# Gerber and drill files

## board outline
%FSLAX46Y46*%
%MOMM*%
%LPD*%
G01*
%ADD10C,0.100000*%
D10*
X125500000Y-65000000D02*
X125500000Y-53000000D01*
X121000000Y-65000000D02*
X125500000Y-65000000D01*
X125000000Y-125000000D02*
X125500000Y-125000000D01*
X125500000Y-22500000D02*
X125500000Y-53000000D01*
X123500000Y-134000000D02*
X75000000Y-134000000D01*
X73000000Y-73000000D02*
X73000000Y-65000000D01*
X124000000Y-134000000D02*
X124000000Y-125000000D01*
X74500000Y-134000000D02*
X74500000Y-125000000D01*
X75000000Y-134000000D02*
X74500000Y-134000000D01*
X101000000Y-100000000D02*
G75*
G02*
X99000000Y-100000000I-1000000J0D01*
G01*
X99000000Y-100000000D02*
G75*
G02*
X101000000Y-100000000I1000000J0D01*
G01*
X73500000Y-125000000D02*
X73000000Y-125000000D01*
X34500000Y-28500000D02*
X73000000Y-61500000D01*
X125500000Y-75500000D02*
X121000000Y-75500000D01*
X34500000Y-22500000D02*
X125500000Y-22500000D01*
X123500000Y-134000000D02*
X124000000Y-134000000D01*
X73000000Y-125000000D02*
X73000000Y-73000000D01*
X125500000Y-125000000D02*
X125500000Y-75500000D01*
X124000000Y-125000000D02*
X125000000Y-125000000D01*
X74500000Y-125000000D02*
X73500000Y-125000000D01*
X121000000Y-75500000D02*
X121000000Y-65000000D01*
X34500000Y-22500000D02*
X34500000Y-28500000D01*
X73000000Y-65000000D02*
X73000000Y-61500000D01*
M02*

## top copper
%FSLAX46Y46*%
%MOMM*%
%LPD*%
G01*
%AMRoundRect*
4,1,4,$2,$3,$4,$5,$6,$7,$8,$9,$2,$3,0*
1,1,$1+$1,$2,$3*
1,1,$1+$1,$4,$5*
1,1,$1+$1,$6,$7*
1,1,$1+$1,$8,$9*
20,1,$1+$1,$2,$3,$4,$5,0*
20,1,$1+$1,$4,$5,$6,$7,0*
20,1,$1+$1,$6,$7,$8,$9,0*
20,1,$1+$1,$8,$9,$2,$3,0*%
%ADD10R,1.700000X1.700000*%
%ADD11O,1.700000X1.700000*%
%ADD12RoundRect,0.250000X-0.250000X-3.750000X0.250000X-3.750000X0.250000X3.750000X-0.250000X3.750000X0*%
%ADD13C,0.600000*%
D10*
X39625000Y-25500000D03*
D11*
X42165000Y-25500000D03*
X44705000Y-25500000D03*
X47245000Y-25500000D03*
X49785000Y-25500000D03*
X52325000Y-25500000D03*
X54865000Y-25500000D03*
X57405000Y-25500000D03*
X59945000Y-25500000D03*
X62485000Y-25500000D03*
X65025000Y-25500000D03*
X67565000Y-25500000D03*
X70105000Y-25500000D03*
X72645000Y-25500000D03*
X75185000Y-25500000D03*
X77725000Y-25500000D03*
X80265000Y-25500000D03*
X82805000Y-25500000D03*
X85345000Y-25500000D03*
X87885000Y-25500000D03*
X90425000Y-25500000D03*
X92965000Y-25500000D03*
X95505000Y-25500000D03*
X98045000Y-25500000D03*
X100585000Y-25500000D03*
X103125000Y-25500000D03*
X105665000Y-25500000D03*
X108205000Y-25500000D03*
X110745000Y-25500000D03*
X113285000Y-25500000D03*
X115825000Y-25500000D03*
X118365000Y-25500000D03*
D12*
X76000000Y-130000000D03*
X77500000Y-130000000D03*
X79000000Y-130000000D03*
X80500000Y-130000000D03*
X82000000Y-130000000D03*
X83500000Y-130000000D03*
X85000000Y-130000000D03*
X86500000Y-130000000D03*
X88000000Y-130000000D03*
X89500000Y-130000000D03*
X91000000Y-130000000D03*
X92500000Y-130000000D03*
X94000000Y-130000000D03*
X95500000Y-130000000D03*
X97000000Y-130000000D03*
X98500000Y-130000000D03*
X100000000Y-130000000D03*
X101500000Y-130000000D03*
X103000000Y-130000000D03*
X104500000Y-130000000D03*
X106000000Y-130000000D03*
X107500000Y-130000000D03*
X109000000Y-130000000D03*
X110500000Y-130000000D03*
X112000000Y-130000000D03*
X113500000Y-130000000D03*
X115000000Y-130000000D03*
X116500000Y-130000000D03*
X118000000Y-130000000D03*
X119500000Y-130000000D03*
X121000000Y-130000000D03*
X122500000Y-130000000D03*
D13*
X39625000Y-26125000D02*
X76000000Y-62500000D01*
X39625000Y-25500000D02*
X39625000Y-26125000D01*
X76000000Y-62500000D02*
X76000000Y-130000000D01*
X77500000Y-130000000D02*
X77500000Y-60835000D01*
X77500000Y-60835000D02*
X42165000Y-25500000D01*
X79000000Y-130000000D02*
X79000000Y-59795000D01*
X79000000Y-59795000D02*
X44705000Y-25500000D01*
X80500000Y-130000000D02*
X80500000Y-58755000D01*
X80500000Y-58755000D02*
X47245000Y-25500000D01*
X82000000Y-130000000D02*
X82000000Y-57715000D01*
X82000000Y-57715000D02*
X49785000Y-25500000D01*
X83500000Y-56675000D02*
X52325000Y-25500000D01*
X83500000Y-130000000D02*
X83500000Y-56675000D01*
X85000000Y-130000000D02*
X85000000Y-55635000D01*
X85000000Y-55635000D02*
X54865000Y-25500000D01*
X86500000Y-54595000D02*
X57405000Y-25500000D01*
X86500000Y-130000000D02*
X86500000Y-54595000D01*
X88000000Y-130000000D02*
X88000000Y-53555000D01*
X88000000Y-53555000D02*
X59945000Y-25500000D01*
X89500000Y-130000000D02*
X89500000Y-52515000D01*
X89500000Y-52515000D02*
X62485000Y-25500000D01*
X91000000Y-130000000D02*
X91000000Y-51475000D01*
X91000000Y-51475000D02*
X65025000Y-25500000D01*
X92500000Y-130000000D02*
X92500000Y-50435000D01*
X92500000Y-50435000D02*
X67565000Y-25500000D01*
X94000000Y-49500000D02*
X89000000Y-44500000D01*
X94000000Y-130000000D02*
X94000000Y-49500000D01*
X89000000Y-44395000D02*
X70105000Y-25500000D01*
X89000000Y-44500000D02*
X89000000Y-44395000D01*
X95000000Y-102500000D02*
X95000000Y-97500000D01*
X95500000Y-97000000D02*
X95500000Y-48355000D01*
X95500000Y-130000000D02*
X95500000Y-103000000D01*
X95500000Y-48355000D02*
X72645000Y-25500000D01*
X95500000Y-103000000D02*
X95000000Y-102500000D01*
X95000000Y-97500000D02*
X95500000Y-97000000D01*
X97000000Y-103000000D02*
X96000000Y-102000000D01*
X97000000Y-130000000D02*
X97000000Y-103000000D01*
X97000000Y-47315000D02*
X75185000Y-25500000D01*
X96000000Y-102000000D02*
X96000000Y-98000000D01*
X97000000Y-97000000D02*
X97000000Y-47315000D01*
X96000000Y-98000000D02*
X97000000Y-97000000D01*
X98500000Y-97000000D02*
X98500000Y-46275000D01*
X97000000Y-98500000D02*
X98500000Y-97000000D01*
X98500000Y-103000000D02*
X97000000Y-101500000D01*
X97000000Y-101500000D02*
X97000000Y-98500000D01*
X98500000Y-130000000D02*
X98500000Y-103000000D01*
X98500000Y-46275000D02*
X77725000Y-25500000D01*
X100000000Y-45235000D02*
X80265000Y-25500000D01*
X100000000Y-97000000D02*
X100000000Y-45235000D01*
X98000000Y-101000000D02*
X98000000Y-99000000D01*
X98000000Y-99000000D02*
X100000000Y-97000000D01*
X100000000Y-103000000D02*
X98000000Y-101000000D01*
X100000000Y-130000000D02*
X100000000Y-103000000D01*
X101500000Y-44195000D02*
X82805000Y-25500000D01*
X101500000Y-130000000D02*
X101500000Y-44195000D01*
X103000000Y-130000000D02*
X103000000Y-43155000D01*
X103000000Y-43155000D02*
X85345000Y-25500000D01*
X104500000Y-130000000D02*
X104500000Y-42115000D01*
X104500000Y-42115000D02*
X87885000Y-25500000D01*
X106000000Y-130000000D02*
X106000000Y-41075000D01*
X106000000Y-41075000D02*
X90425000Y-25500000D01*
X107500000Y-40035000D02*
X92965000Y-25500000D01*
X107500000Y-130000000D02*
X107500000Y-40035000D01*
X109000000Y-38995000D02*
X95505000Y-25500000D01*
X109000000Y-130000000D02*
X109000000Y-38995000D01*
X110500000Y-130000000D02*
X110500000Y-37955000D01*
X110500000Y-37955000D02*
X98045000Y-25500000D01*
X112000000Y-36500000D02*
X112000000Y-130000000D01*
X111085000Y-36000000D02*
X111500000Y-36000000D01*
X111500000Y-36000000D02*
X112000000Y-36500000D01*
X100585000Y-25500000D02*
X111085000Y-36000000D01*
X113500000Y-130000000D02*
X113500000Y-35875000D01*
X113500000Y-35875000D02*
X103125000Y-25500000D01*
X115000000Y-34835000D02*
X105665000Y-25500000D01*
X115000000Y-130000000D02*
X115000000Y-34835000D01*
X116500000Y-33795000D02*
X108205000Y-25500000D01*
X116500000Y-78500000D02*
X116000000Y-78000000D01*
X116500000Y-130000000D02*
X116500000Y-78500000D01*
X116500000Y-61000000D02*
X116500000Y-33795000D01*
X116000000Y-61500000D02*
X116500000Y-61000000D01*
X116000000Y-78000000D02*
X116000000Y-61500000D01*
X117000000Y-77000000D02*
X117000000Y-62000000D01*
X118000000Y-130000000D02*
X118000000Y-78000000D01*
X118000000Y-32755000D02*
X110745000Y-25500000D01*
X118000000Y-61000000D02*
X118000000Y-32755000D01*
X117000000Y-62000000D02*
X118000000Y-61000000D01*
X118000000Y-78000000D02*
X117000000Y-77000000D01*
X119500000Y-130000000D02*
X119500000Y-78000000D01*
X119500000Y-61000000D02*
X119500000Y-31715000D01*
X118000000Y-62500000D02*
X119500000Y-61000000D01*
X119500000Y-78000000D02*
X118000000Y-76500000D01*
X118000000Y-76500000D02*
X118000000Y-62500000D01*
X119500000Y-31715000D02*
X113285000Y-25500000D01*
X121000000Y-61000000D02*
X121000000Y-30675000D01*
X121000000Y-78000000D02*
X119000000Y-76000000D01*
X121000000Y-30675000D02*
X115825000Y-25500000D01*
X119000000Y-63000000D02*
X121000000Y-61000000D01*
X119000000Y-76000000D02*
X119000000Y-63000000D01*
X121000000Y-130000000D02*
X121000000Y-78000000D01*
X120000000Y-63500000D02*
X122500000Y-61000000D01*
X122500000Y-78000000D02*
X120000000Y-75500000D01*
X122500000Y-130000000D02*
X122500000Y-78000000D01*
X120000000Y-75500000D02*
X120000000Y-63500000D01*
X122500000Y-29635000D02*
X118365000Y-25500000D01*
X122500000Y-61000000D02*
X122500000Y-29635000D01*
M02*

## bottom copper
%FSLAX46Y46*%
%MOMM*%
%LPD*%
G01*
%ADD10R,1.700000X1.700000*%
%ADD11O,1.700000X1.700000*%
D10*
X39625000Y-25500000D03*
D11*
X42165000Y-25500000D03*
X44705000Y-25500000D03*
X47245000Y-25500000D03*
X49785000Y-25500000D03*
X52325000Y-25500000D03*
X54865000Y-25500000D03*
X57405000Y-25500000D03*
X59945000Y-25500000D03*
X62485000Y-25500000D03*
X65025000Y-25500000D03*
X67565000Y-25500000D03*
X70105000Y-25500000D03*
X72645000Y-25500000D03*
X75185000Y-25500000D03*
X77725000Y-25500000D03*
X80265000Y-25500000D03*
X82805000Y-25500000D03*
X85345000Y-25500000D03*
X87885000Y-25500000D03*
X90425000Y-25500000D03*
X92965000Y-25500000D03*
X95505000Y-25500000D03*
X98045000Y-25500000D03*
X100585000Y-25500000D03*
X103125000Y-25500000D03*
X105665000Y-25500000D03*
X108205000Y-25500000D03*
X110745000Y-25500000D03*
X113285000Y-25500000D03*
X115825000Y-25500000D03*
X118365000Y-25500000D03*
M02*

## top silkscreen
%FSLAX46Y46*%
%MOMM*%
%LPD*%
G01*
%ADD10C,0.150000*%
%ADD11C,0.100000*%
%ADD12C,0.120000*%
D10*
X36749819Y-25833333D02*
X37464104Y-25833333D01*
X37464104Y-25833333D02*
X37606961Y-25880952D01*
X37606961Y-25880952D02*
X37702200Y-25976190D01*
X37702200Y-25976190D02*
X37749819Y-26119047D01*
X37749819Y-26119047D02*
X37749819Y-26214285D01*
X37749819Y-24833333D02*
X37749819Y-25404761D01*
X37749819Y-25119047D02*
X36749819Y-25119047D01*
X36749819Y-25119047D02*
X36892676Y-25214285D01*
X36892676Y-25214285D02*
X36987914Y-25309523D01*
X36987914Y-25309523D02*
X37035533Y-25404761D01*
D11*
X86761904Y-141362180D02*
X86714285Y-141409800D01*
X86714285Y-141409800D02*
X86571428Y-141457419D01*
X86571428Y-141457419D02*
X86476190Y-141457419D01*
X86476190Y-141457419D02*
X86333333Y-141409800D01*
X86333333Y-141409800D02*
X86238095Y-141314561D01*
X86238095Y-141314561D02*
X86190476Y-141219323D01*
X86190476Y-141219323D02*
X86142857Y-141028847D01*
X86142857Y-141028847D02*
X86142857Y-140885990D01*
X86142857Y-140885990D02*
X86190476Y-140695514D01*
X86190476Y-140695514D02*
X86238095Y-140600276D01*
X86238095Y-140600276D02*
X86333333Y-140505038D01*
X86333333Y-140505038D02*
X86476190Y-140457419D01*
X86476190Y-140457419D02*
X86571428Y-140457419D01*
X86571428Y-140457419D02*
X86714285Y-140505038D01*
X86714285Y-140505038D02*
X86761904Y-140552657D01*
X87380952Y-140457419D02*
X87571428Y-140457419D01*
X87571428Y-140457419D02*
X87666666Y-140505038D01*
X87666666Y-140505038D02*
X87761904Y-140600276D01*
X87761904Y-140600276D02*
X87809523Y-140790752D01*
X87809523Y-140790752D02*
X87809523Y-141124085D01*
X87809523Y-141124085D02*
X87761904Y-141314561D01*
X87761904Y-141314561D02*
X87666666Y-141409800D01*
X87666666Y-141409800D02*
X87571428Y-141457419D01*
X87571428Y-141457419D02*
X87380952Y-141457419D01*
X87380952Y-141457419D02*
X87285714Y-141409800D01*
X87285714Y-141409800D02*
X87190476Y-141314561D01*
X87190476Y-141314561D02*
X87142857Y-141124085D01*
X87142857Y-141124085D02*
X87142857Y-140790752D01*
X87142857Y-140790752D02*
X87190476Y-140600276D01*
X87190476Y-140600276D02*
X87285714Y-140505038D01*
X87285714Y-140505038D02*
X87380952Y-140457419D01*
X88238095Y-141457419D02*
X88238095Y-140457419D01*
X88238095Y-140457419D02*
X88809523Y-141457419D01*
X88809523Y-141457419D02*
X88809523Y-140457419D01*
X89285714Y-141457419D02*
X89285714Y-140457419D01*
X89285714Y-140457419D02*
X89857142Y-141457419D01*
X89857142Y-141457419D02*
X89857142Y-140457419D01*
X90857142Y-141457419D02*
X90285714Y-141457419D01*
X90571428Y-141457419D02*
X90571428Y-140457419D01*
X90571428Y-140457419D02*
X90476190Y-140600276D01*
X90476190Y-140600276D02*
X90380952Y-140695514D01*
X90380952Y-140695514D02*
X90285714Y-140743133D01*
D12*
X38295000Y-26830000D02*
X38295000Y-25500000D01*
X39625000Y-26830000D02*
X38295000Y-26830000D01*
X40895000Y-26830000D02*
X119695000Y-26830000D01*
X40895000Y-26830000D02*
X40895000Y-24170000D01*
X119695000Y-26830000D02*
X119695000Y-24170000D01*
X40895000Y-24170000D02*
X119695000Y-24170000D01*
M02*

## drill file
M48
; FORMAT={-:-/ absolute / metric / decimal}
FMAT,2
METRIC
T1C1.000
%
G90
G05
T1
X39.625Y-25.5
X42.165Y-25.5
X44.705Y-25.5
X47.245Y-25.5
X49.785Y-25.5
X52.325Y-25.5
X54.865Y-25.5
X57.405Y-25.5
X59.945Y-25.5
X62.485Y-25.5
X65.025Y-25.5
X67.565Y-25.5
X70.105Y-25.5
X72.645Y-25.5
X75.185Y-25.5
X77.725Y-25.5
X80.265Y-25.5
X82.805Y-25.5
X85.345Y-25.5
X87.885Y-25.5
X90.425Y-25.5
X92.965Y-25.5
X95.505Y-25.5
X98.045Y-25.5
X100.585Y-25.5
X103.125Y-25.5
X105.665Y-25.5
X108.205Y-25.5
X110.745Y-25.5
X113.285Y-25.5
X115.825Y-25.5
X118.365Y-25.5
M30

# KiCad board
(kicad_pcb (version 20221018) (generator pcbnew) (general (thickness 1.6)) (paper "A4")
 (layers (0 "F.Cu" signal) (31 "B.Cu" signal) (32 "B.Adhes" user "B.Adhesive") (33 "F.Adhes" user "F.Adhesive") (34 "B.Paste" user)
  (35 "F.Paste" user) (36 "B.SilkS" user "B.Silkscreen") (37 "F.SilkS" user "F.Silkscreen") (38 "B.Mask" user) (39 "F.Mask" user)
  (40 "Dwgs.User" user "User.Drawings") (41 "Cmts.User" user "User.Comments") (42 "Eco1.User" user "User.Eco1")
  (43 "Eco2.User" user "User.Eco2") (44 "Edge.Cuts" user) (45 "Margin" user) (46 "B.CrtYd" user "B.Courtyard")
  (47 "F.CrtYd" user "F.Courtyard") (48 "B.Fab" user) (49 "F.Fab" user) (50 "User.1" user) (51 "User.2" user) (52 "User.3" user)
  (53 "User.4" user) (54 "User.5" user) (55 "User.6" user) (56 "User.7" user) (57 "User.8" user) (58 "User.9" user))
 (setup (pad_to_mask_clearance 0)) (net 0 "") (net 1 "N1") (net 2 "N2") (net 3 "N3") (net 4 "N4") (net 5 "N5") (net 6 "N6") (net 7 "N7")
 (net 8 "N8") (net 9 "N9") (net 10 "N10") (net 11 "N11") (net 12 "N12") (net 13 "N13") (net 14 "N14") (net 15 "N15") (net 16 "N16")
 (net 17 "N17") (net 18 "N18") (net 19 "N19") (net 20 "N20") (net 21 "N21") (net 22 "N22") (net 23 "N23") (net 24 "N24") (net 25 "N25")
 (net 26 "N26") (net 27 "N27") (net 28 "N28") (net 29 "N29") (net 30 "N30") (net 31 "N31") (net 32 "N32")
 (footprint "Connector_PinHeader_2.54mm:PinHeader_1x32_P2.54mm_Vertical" (layer "F.Cu") (at 39.625 25.5 90)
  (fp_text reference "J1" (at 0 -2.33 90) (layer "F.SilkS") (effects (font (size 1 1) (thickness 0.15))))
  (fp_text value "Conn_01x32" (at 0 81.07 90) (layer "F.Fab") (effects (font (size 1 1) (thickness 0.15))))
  (fp_line (start -1.33 -1.33) (end 0 -1.33) (stroke (width 0.12) (type solid)) (layer "F.SilkS"))
  (fp_line (start -1.33 0) (end -1.33 -1.33) (stroke (width 0.12) (type solid)) (layer "F.SilkS"))
  (fp_line (start -1.33 1.27) (end -1.33 80.07) (stroke (width 0.12) (type solid)) (layer "F.SilkS"))
  (fp_line (start -1.33 1.27) (end 1.33 1.27) (stroke (width 0.12) (type solid)) (layer "F.SilkS"))
  (fp_line (start -1.33 80.07) (end 1.33 80.07) (stroke (width 0.12) (type solid)) (layer "F.SilkS"))
  (fp_line (start 1.33 1.27) (end 1.33 80.07) (stroke (width 0.12) (type solid)) (layer "F.SilkS"))
  (pad "1" thru_hole rect (at 0 0 90) (size 1.7 1.7) (drill 1) (layers "*.Cu" "*.Mask") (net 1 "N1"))
  (pad "2" thru_hole oval (at 0 2.54 90) (size 1.7 1.7) (drill 1) (layers "*.Cu" "*.Mask") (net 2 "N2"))
  (pad "3" thru_hole oval (at 0 5.08 90) (size 1.7 1.7) (drill 1) (layers "*.Cu" "*.Mask") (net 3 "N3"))
  (pad "4" thru_hole oval (at 0 7.62 90) (size 1.7 1.7) (drill 1) (layers "*.Cu" "*.Mask") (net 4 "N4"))
  (pad "5" thru_hole oval (at 0 10.16 90) (size 1.7 1.7) (drill 1) (layers "*.Cu" "*.Mask") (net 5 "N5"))
  (pad "6" thru_hole oval (at 0 12.7 90) (size 1.7 1.7) (drill 1) (layers "*.Cu" "*.Mask") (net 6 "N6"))
  (pad "7" thru_hole oval (at 0 15.24 90) (size 1.7 1.7) (drill 1) (layers "*.Cu" "*.Mask") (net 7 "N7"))
  (pad "8" thru_hole oval (at 0 17.78 90) (size 1.7 1.7) (drill 1) (layers "*.Cu" "*.Mask") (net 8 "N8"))
  (pad "9" thru_hole oval (at 0 20.32 90) (size 1.7 1.7) (drill 1) (layers "*.Cu" "*.Mask") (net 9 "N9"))
  (pad "10" thru_hole oval (at 0 22.86 90) (size 1.7 1.7) (drill 1) (layers "*.Cu" "*.Mask") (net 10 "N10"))
  (pad "11" thru_hole oval (at 0 25.4 90) (size 1.7 1.7) (drill 1) (layers "*.Cu" "*.Mask") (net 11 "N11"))
  (pad "12" thru_hole oval (at 0 27.94 90) (size 1.7 1.7) (drill 1) (layers "*.Cu" "*.Mask") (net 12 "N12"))
  (pad "13" thru_hole oval (at 0 30.48 90) (size 1.7 1.7) (drill 1) (layers "*.Cu" "*.Mask") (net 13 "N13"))
  (pad "14" thru_hole oval (at 0 33.02 90) (size 1.7 1.7) (drill 1) (layers "*.Cu" "*.Mask") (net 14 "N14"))
  (pad "15" thru_hole oval (at 0 35.56 90) (size 1.7 1.7) (drill 1) (layers "*.Cu" "*.Mask") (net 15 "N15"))
  (pad "16" thru_hole oval (at 0 38.1 90) (size 1.7 1.7) (drill 1) (layers "*.Cu" "*.Mask") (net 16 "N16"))
  (pad "17" thru_hole oval (at 0 40.64 90) (size 1.7 1.7) (drill 1) (layers "*.Cu" "*.Mask") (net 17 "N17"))
  (pad "18" thru_hole oval (at 0 43.18 90) (size 1.7 1.7) (drill 1) (layers "*.Cu" "*.Mask") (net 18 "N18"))
  (pad "19" thru_hole oval (at 0 45.72 90) (size 1.7 1.7) (drill 1) (layers "*.Cu" "*.Mask") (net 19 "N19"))
  (pad "20" thru_hole oval (at 0 48.26 90) (size 1.7 1.7) (drill 1) (layers "*.Cu" "*.Mask") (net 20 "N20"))
  (pad "21" thru_hole oval (at 0 50.8 90) (size 1.7 1.7) (drill 1) (layers "*.Cu" "*.Mask") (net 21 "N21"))
  (pad "22" thru_hole oval (at 0 53.34 90) (size 1.7 1.7) (drill 1) (layers "*.Cu" "*.Mask") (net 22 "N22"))
  (pad "23" thru_hole oval (at 0 55.88 90) (size 1.7 1.7) (drill 1) (layers "*.Cu" "*.Mask") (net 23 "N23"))
  (pad "24" thru_hole oval (at 0 58.42 90) (size 1.7 1.7) (drill 1) (layers "*.Cu" "*.Mask") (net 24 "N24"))
  (pad "25" thru_hole oval (at 0 60.96 90) (size 1.7 1.7) (drill 1) (layers "*.Cu" "*.Mask") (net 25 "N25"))
  (pad "26" thru_hole oval (at 0 63.5 90) (size 1.7 1.7) (drill 1) (layers "*.Cu" "*.Mask") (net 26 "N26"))
  (pad "27" thru_hole oval (at 0 66.04 90) (size 1.7 1.7) (drill 1) (layers "*.Cu" "*.Mask") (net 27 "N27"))
  (pad "28" thru_hole oval (at 0 68.58 90) (size 1.7 1.7) (drill 1) (layers "*.Cu" "*.Mask") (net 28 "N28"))
  (pad "29" thru_hole oval (at 0 71.12 90) (size 1.7 1.7) (drill 1) (layers "*.Cu" "*.Mask") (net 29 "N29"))
  (pad "30" thru_hole oval (at 0 73.66 90) (size 1.7 1.7) (drill 1) (layers "*.Cu" "*.Mask") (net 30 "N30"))
  (pad "31" thru_hole oval (at 0 76.2 90) (size 1.7 1.7) (drill 1) (layers "*.Cu" "*.Mask") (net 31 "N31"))
  (pad "32" thru_hole oval (at 0 78.74 90) (size 1.7 1.7) (drill 1) (layers "*.Cu" "*.Mask") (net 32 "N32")))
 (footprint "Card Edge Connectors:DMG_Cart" (layer "F.Cu") (at 75 134)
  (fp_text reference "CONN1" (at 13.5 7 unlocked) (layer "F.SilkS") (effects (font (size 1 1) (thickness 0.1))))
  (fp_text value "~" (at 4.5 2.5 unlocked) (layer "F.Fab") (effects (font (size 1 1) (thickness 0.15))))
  (pad "1" smd roundrect (at 1 -4) (size 1 8) (layers "F.Cu" "F.Paste" "F.Mask") (roundrect_rratio 0.25) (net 1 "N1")
   (thermal_bridge_angle 45))
  (pad "2" smd roundrect (at 2.5 -4) (size 1 8) (layers "F.Cu" "F.Paste" "F.Mask") (roundrect_rratio 0.25) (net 2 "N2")
   (thermal_bridge_angle 45))
  (pad "3" smd roundrect (at 4 -4) (size 1 8) (layers "F.Cu" "F.Paste" "F.Mask") (roundrect_rratio 0.25) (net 3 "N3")
   (thermal_bridge_angle 45))
  (pad "4" smd roundrect (at 5.5 -4) (size 1 8) (layers "F.Cu" "F.Paste" "F.Mask") (roundrect_rratio 0.25) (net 4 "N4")
   (thermal_bridge_angle 45))
  (pad "5" smd roundrect (at 7 -4) (size 1 8) (layers "F.Cu" "F.Paste" "F.Mask") (roundrect_rratio 0.25) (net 5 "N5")
   (thermal_bridge_angle 45))
  (pad "6" smd roundrect (at 8.5 -4) (size 1 8) (layers "F.Cu" "F.Paste" "F.Mask") (roundrect_rratio 0.25) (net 6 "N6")
   (thermal_bridge_angle 45))
  (pad "7" smd roundrect (at 10 -4) (size 1 8) (layers "F.Cu" "F.Paste" "F.Mask") (roundrect_rratio 0.25) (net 7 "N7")
   (thermal_bridge_angle 45))
  (pad "8" smd roundrect (at 11.5 -4) (size 1 8) (layers "F.Cu" "F.Paste" "F.Mask") (roundrect_rratio 0.25) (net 8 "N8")
   (thermal_bridge_angle 45))
  (pad "9" smd roundrect (at 13 -4) (size 1 8) (layers "F.Cu" "F.Paste" "F.Mask") (roundrect_rratio 0.25) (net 9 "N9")
   (thermal_bridge_angle 45))
  (pad "10" smd roundrect (at 14.5 -4) (size 1 8) (layers "F.Cu" "F.Paste" "F.Mask") (roundrect_rratio 0.25) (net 10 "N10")
   (thermal_bridge_angle 45))
  (pad "11" smd roundrect (at 16 -4) (size 1 8) (layers "F.Cu" "F.Paste" "F.Mask") (roundrect_rratio 0.25) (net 11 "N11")
   (thermal_bridge_angle 45))
  (pad "12" smd roundrect (at 17.5 -4) (size 1 8) (layers "F.Cu" "F.Paste" "F.Mask") (roundrect_rratio 0.25) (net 12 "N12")
   (thermal_bridge_angle 45))
  (pad "13" smd roundrect (at 19 -4) (size 1 8) (layers "F.Cu" "F.Paste" "F.Mask") (roundrect_rratio 0.25) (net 13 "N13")
   (thermal_bridge_angle 45))
  (pad "14" smd roundrect (at 20.5 -4) (size 1 8) (layers "F.Cu" "F.Paste" "F.Mask") (roundrect_rratio 0.25) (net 14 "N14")
   (thermal_bridge_angle 45))
  (pad "15" smd roundrect (at 22 -4) (size 1 8) (layers "F.Cu" "F.Paste" "F.Mask") (roundrect_rratio 0.25) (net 15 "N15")
   (thermal_bridge_angle 45))
  (pad "16" smd roundrect (at 23.5 -4) (size 1 8) (layers "F.Cu" "F.Paste" "F.Mask") (roundrect_rratio 0.25) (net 16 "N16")
   (thermal_bridge_angle 45))
  (pad "17" smd roundrect (at 25 -4) (size 1 8) (layers "F.Cu" "F.Paste" "F.Mask") (roundrect_rratio 0.25) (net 17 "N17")
   (thermal_bridge_angle 45))
  (pad "18" smd roundrect (at 26.5 -4) (size 1 8) (layers "F.Cu" "F.Paste" "F.Mask") (roundrect_rratio 0.25) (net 18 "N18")
   (thermal_bridge_angle 45))
  (pad "19" smd roundrect (at 28 -4) (size 1 8) (layers "F.Cu" "F.Paste" "F.Mask") (roundrect_rratio 0.25) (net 19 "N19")
   (thermal_bridge_angle 45))
  (pad "20" smd roundrect (at 29.5 -4) (size 1 8) (layers "F.Cu" "F.Paste" "F.Mask") (roundrect_rratio 0.25) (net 20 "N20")
   (thermal_bridge_angle 45))
  (pad "21" smd roundrect (at 31 -4) (size 1 8) (layers "F.Cu" "F.Paste" "F.Mask") (roundrect_rratio 0.25) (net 21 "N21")
   (thermal_bridge_angle 45))
  (pad "22" smd roundrect (at 32.5 -4) (size 1 8) (layers "F.Cu" "F.Paste" "F.Mask") (roundrect_rratio 0.25) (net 22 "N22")
   (thermal_bridge_angle 45))
  (pad "23" smd roundrect (at 34 -4) (size 1 8) (layers "F.Cu" "F.Paste" "F.Mask") (roundrect_rratio 0.25) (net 23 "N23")
   (thermal_bridge_angle 45))
  (pad "24" smd roundrect (at 35.5 -4) (size 1 8) (layers "F.Cu" "F.Paste" "F.Mask") (roundrect_rratio 0.25) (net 24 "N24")
   (thermal_bridge_angle 45))
  (pad "25" smd roundrect (at 37 -4) (size 1 8) (layers "F.Cu" "F.Paste" "F.Mask") (roundrect_rratio 0.25) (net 25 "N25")
   (thermal_bridge_angle 45))
  (pad "26" smd roundrect (at 38.5 -4) (size 1 8) (layers "F.Cu" "F.Paste" "F.Mask") (roundrect_rratio 0.25) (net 26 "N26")
   (thermal_bridge_angle 45))
  (pad "27" smd roundrect (at 40 -4) (size 1 8) (layers "F.Cu" "F.Paste" "F.Mask") (roundrect_rratio 0.25) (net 27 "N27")
   (thermal_bridge_angle 45))
  (pad "28" smd roundrect (at 41.5 -4) (size 1 8) (layers "F.Cu" "F.Paste" "F.Mask") (roundrect_rratio 0.25) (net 28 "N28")
   (thermal_bridge_angle 45))
  (pad "29" smd roundrect (at 43 -4) (size 1 8) (layers "F.Cu" "F.Paste" "F.Mask") (roundrect_rratio 0.25) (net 29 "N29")
   (thermal_bridge_angle 45))
  (pad "30" smd roundrect (at 44.5 -4) (size 1 8) (layers "F.Cu" "F.Paste" "F.Mask") (roundrect_rratio 0.25) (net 30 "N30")
   (thermal_bridge_angle 45))
  (pad "31" smd roundrect (at 46 -4) (size 1 8) (layers "F.Cu" "F.Paste" "F.Mask") (roundrect_rratio 0.25) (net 31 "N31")
   (thermal_bridge_angle 45))
  (pad "32" smd roundrect (at 47.5 -4) (size 1 8) (layers "F.Cu" "F.Paste" "F.Mask") (roundrect_rratio 0.25) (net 32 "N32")
   (thermal_bridge_angle 45)))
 (gr_line (start 125.5 65) (end 125.5 53) (stroke (width 0.1) (type default)) (layer "Edge.Cuts"))
 (gr_line (start 121 65) (end 125.5 65) (stroke (width 0.1) (type default)) (layer "Edge.Cuts"))
 (gr_line (start 125 125) (end 125.5 125) (stroke (width 0.1) (type default)) (layer "Edge.Cuts"))
 (gr_line (start 125.5 22.5) (end 125.5 53) (stroke (width 0.1) (type default)) (layer "Edge.Cuts"))
 (gr_line (start 123.5 134) (end 75 134) (stroke (width 0.1) (type default)) (layer "Edge.Cuts"))
 (gr_line (start 73 73) (end 73 65) (stroke (width 0.1) (type default)) (layer "Edge.Cuts"))
 (gr_line (start 124 134) (end 124 125) (stroke (width 0.1) (type default)) (layer "Edge.Cuts"))
 (gr_line (start 74.5 134) (end 74.5 125) (stroke (width 0.1) (type default)) (layer "Edge.Cuts"))
 (gr_line (start 75 134) (end 74.5 134) (stroke (width 0.1) (type default)) (layer "Edge.Cuts"))
 (gr_circle (center 100 100) (end 101 100) (stroke (width 0.1) (type default)) (fill none) (layer "Edge.Cuts"))
 (gr_line (start 73.5 125) (end 73 125) (stroke (width 0.1) (type default)) (layer "Edge.Cuts"))
 (gr_line (start 34.5 28.5) (end 73 61.5) (stroke (width 0.1) (type default)) (layer "Edge.Cuts"))
 (gr_line (start 125.5 75.5) (end 121 75.5) (stroke (width 0.1) (type default)) (layer "Edge.Cuts"))
 (gr_line (start 34.5 22.5) (end 125.5 22.5) (stroke (width 0.1) (type default)) (layer "Edge.Cuts"))
 (gr_line (start 123.5 134) (end 124 134) (stroke (width 0.1) (type default)) (layer "Edge.Cuts"))
 (gr_line (start 73 125) (end 73 73) (stroke (width 0.1) (type default)) (layer "Edge.Cuts"))
 (gr_line (start 125.5 125) (end 125.5 75.5) (stroke (width 0.1) (type default)) (layer "Edge.Cuts"))
 (gr_line (start 124 125) (end 125 125) (stroke (width 0.1) (type default)) (layer "Edge.Cuts"))
 (gr_line (start 74.5 125) (end 73.5 125) (stroke (width 0.1) (type default)) (layer "Edge.Cuts"))
 (gr_line (start 121 75.5) (end 121 65) (stroke (width 0.1) (type default)) (layer "Edge.Cuts"))
 (gr_line (start 34.5 22.5) (end 34.5 28.5) (stroke (width 0.1) (type default)) (layer "Edge.Cuts"))
 (gr_line (start 73 65) (end 73 61.5) (stroke (width 0.1) (type default)) (layer "Edge.Cuts"))
 (segment (start 39.625 26.125) (end 76 62.5) (width 0.6) (layer "F.Cu") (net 1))
 (segment (start 39.625 25.5) (end 39.625 26.125) (width 0.6) (layer "F.Cu") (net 1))
 (segment (start 76 62.5) (end 76 130) (width 0.6) (layer "F.Cu") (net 1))
 (segment (start 77.5 130) (end 77.5 60.835) (width 0.6) (layer "F.Cu") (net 2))
 (segment (start 77.5 60.835) (end 42.165 25.5) (width 0.6) (layer "F.Cu") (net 2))
 (segment (start 79 130) (end 79 59.795) (width 0.6) (layer "F.Cu") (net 3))
 (segment (start 79 59.795) (end 44.705 25.5) (width 0.6) (layer "F.Cu") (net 3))
 (segment (start 80.5 130) (end 80.5 58.755) (width 0.6) (layer "F.Cu") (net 4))
 (segment (start 80.5 58.755) (end 47.245 25.5) (width 0.6) (layer "F.Cu") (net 4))
 (segment (start 82 130) (end 82 57.715) (width 0.6) (layer "F.Cu") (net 5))
 (segment (start 82 57.715) (end 49.785 25.5) (width 0.6) (layer "F.Cu") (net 5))
 (segment (start 83.5 56.675) (end 52.325 25.5) (width 0.6) (layer "F.Cu") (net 6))
 (segment (start 83.5 130) (end 83.5 56.675) (width 0.6) (layer "F.Cu") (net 6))
 (segment (start 85 130) (end 85 55.635) (width 0.6) (layer "F.Cu") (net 7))
 (segment (start 85 55.635) (end 54.865 25.5) (width 0.6) (layer "F.Cu") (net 7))
 (segment (start 86.5 54.595) (end 57.405 25.5) (width 0.6) (layer "F.Cu") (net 8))
 (segment (start 86.5 130) (end 86.5 54.595) (width 0.6) (layer "F.Cu") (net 8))
 (segment (start 88 130) (end 88 53.555) (width 0.6) (layer "F.Cu") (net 9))
 (segment (start 88 53.555) (end 59.945 25.5) (width 0.6) (layer "F.Cu") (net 9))
 (segment (start 89.5 130) (end 89.5 52.515) (width 0.6) (layer "F.Cu") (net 10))
 (segment (start 89.5 52.515) (end 62.485 25.5) (width 0.6) (layer "F.Cu") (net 10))
 (segment (start 91 130) (end 91 51.475) (width 0.6) (layer "F.Cu") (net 11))
 (segment (start 91 51.475) (end 65.025 25.5) (width 0.6) (layer "F.Cu") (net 11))
 (segment (start 92.5 130) (end 92.5 50.435) (width 0.6) (layer "F.Cu") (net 12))
 (segment (start 92.5 50.435) (end 67.565 25.5) (width 0.6) (layer "F.Cu") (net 12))
 (segment (start 94 49.5) (end 89 44.5) (width 0.6) (layer "F.Cu") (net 13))
 (segment (start 94 130) (end 94 49.5) (width 0.6) (layer "F.Cu") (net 13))
 (segment (start 89 44.395) (end 70.105 25.5) (width 0.6) (layer "F.Cu") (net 13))
 (segment (start 89 44.5) (end 89 44.395) (width 0.6) (layer "F.Cu") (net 13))
 (segment (start 95 102.5) (end 95 97.5) (width 0.6) (layer "F.Cu") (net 14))
 (segment (start 95.5 97) (end 95.5 48.355) (width 0.6) (layer "F.Cu") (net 14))
 (segment (start 95.5 130) (end 95.5 103) (width 0.6) (layer "F.Cu") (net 14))
 (segment (start 95.5 48.355) (end 72.645 25.5) (width 0.6) (layer "F.Cu") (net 14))
 (segment (start 95.5 103) (end 95 102.5) (width 0.6) (layer "F.Cu") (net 14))
 (segment (start 95 97.5) (end 95.5 97) (width 0.6) (layer "F.Cu") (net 14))
 (segment (start 97 103) (end 96 102) (width 0.6) (layer "F.Cu") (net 15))
 (segment (start 97 130) (end 97 103) (width 0.6) (layer "F.Cu") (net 15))
 (segment (start 97 47.315) (end 75.185 25.5) (width 0.6) (layer "F.Cu") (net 15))
 (segment (start 96 102) (end 96 98) (width 0.6) (layer "F.Cu") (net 15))
 (segment (start 97 97) (end 97 47.315) (width 0.6) (layer "F.Cu") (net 15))
 (segment (start 96 98) (end 97 97) (width 0.6) (layer "F.Cu") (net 15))
 (segment (start 98.5 97) (end 98.5 46.275) (width 0.6) (layer "F.Cu") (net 16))
 (segment (start 97 98.5) (end 98.5 97) (width 0.6) (layer "F.Cu") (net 16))
 (segment (start 98.5 103) (end 97 101.5) (width 0.6) (layer "F.Cu") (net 16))
 (segment (start 97 101.5) (end 97 98.5) (width 0.6) (layer "F.Cu") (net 16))
 (segment (start 98.5 130) (end 98.5 103) (width 0.6) (layer "F.Cu") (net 16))
 (segment (start 98.5 46.275) (end 77.725 25.5) (width 0.6) (layer "F.Cu") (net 16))
 (segment (start 100 45.235) (end 80.265 25.5) (width 0.6) (layer "F.Cu") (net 17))
 (segment (start 100 97) (end 100 45.235) (width 0.6) (layer "F.Cu") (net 17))
 (segment (start 98 101) (end 98 99) (width 0.6) (layer "F.Cu") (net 17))
 (segment (start 98 99) (end 100 97) (width 0.6) (layer "F.Cu") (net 17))
 (segment (start 100 103) (end 98 101) (width 0.6) (layer "F.Cu") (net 17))
 (segment (start 100 130) (end 100 103) (width 0.6) (layer "F.Cu") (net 17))
 (segment (start 101.5 44.195) (end 82.805 25.5) (width 0.6) (layer "F.Cu") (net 18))
 (segment (start 101.5 130) (end 101.5 44.195) (width 0.6) (layer "F.Cu") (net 18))
 (segment (start 103 130) (end 103 43.155) (width 0.6) (layer "F.Cu") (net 19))
 (segment (start 103 43.155) (end 85.345 25.5) (width 0.6) (layer "F.Cu") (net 19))
 (segment (start 104.5 130) (end 104.5 42.115) (width 0.6) (layer "F.Cu") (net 20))
 (segment (start 104.5 42.115) (end 87.885 25.5) (width 0.6) (layer "F.Cu") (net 20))
 (segment (start 106 130) (end 106 41.075) (width 0.6) (layer "F.Cu") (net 21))
 (segment (start 106 41.075) (end 90.425 25.5) (width 0.6) (layer "F.Cu") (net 21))
 (segment (start 107.5 40.035) (end 92.965 25.5) (width 0.6) (layer "F.Cu") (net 22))
 (segment (start 107.5 130) (end 107.5 40.035) (width 0.6) (layer "F.Cu") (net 22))
 (segment (start 109 38.995) (end 95.505 25.5) (width 0.6) (layer "F.Cu") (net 23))
 (segment (start 109 130) (end 109 38.995) (width 0.6) (layer "F.Cu") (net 23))
 (segment (start 110.5 130) (end 110.5 37.955) (width 0.6) (layer "F.Cu") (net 24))
 (segment (start 110.5 37.955) (end 98.045 25.5) (width 0.6) (layer "F.Cu") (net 24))
 (segment (start 112 36.5) (end 112 130) (width 0.6) (layer "F.Cu") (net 25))
 (segment (start 111.085 36) (end 111.5 36) (width 0.6) (layer "F.Cu") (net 25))
 (segment (start 111.5 36) (end 112 36.5) (width 0.6) (layer "F.Cu") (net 25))
 (segment (start 100.585 25.5) (end 111.085 36) (width 0.6) (layer "F.Cu") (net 25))
 (segment (start 113.5 130) (end 113.5 35.875) (width 0.6) (layer "F.Cu") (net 26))
 (segment (start 113.5 35.875) (end 103.125 25.5) (width 0.6) (layer "F.Cu") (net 26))
 (segment (start 115 34.835) (end 105.665 25.5) (width 0.6) (layer "F.Cu") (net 27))
 (segment (start 115 130) (end 115 34.835) (width 0.6) (layer "F.Cu") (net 27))
 (segment (start 116.5 33.795) (end 108.205 25.5) (width 0.6) (layer "F.Cu") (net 28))
 (segment (start 116.5 78.5) (end 116 78) (width 0.6) (layer "F.Cu") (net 28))
 (segment (start 116.5 130) (end 116.5 78.5) (width 0.6) (layer "F.Cu") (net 28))
 (segment (start 116.5 61) (end 116.5 33.795) (width 0.6) (layer "F.Cu") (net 28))
 (segment (start 116 61.5) (end 116.5 61) (width 0.6) (layer "F.Cu") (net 28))
 (segment (start 116 78) (end 116 61.5) (width 0.6) (layer "F.Cu") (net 28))
 (segment (start 117 77) (end 117 62) (width 0.6) (layer "F.Cu") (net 29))
 (segment (start 118 130) (end 118 78) (width 0.6) (layer "F.Cu") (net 29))
 (segment (start 118 32.755) (end 110.745 25.5) (width 0.6) (layer "F.Cu") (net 29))
 (segment (start 118 61) (end 118 32.755) (width 0.6) (layer "F.Cu") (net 29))
 (segment (start 117 62) (end 118 61) (width 0.6) (layer "F.Cu") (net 29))
 (segment (start 118 78) (end 117 77) (width 0.6) (layer "F.Cu") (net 29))
 (segment (start 119.5 130) (end 119.5 78) (width 0.6) (layer "F.Cu") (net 30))
 (segment (start 119.5 61) (end 119.5 31.715) (width 0.6) (layer "F.Cu") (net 30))
 (segment (start 118 62.5) (end 119.5 61) (width 0.6) (layer "F.Cu") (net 30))
 (segment (start 119.5 78) (end 118 76.5) (width 0.6) (layer "F.Cu") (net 30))
 (segment (start 118 76.5) (end 118 62.5) (width 0.6) (layer "F.Cu") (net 30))
 (segment (start 119.5 31.715) (end 113.285 25.5) (width 0.6) (layer "F.Cu") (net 30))
 (segment (start 121 61) (end 121 30.675) (width 0.6) (layer "F.Cu") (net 31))
 (segment (start 121 78) (end 119 76) (width 0.6) (layer "F.Cu") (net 31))
 (segment (start 121 30.675) (end 115.825 25.5) (width 0.6) (layer "F.Cu") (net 31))
 (segment (start 119 63) (end 121 61) (width 0.6) (layer "F.Cu") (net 31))
 (segment (start 119 76) (end 119 63) (width 0.6) (layer "F.Cu") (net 31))
 (segment (start 121 130) (end 121 78) (width 0.6) (layer "F.Cu") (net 31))
 (segment (start 120 63.5) (end 122.5 61) (width 0.6) (layer "F.Cu") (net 32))
 (segment (start 122.5 78) (end 120 75.5) (width 0.6) (layer "F.Cu") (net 32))
 (segment (start 122.5 130) (end 122.5 78) (width 0.6) (layer "F.Cu") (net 32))
 (segment (start 120 75.5) (end 120 63.5) (width 0.6) (layer "F.Cu") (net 32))
 (segment (start 122.5 29.635) (end 118.365 25.5) (width 0.6) (layer "F.Cu") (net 32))
 (segment (start 122.5 61) (end 122.5 29.635) (width 0.6) (layer "F.Cu") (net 32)))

